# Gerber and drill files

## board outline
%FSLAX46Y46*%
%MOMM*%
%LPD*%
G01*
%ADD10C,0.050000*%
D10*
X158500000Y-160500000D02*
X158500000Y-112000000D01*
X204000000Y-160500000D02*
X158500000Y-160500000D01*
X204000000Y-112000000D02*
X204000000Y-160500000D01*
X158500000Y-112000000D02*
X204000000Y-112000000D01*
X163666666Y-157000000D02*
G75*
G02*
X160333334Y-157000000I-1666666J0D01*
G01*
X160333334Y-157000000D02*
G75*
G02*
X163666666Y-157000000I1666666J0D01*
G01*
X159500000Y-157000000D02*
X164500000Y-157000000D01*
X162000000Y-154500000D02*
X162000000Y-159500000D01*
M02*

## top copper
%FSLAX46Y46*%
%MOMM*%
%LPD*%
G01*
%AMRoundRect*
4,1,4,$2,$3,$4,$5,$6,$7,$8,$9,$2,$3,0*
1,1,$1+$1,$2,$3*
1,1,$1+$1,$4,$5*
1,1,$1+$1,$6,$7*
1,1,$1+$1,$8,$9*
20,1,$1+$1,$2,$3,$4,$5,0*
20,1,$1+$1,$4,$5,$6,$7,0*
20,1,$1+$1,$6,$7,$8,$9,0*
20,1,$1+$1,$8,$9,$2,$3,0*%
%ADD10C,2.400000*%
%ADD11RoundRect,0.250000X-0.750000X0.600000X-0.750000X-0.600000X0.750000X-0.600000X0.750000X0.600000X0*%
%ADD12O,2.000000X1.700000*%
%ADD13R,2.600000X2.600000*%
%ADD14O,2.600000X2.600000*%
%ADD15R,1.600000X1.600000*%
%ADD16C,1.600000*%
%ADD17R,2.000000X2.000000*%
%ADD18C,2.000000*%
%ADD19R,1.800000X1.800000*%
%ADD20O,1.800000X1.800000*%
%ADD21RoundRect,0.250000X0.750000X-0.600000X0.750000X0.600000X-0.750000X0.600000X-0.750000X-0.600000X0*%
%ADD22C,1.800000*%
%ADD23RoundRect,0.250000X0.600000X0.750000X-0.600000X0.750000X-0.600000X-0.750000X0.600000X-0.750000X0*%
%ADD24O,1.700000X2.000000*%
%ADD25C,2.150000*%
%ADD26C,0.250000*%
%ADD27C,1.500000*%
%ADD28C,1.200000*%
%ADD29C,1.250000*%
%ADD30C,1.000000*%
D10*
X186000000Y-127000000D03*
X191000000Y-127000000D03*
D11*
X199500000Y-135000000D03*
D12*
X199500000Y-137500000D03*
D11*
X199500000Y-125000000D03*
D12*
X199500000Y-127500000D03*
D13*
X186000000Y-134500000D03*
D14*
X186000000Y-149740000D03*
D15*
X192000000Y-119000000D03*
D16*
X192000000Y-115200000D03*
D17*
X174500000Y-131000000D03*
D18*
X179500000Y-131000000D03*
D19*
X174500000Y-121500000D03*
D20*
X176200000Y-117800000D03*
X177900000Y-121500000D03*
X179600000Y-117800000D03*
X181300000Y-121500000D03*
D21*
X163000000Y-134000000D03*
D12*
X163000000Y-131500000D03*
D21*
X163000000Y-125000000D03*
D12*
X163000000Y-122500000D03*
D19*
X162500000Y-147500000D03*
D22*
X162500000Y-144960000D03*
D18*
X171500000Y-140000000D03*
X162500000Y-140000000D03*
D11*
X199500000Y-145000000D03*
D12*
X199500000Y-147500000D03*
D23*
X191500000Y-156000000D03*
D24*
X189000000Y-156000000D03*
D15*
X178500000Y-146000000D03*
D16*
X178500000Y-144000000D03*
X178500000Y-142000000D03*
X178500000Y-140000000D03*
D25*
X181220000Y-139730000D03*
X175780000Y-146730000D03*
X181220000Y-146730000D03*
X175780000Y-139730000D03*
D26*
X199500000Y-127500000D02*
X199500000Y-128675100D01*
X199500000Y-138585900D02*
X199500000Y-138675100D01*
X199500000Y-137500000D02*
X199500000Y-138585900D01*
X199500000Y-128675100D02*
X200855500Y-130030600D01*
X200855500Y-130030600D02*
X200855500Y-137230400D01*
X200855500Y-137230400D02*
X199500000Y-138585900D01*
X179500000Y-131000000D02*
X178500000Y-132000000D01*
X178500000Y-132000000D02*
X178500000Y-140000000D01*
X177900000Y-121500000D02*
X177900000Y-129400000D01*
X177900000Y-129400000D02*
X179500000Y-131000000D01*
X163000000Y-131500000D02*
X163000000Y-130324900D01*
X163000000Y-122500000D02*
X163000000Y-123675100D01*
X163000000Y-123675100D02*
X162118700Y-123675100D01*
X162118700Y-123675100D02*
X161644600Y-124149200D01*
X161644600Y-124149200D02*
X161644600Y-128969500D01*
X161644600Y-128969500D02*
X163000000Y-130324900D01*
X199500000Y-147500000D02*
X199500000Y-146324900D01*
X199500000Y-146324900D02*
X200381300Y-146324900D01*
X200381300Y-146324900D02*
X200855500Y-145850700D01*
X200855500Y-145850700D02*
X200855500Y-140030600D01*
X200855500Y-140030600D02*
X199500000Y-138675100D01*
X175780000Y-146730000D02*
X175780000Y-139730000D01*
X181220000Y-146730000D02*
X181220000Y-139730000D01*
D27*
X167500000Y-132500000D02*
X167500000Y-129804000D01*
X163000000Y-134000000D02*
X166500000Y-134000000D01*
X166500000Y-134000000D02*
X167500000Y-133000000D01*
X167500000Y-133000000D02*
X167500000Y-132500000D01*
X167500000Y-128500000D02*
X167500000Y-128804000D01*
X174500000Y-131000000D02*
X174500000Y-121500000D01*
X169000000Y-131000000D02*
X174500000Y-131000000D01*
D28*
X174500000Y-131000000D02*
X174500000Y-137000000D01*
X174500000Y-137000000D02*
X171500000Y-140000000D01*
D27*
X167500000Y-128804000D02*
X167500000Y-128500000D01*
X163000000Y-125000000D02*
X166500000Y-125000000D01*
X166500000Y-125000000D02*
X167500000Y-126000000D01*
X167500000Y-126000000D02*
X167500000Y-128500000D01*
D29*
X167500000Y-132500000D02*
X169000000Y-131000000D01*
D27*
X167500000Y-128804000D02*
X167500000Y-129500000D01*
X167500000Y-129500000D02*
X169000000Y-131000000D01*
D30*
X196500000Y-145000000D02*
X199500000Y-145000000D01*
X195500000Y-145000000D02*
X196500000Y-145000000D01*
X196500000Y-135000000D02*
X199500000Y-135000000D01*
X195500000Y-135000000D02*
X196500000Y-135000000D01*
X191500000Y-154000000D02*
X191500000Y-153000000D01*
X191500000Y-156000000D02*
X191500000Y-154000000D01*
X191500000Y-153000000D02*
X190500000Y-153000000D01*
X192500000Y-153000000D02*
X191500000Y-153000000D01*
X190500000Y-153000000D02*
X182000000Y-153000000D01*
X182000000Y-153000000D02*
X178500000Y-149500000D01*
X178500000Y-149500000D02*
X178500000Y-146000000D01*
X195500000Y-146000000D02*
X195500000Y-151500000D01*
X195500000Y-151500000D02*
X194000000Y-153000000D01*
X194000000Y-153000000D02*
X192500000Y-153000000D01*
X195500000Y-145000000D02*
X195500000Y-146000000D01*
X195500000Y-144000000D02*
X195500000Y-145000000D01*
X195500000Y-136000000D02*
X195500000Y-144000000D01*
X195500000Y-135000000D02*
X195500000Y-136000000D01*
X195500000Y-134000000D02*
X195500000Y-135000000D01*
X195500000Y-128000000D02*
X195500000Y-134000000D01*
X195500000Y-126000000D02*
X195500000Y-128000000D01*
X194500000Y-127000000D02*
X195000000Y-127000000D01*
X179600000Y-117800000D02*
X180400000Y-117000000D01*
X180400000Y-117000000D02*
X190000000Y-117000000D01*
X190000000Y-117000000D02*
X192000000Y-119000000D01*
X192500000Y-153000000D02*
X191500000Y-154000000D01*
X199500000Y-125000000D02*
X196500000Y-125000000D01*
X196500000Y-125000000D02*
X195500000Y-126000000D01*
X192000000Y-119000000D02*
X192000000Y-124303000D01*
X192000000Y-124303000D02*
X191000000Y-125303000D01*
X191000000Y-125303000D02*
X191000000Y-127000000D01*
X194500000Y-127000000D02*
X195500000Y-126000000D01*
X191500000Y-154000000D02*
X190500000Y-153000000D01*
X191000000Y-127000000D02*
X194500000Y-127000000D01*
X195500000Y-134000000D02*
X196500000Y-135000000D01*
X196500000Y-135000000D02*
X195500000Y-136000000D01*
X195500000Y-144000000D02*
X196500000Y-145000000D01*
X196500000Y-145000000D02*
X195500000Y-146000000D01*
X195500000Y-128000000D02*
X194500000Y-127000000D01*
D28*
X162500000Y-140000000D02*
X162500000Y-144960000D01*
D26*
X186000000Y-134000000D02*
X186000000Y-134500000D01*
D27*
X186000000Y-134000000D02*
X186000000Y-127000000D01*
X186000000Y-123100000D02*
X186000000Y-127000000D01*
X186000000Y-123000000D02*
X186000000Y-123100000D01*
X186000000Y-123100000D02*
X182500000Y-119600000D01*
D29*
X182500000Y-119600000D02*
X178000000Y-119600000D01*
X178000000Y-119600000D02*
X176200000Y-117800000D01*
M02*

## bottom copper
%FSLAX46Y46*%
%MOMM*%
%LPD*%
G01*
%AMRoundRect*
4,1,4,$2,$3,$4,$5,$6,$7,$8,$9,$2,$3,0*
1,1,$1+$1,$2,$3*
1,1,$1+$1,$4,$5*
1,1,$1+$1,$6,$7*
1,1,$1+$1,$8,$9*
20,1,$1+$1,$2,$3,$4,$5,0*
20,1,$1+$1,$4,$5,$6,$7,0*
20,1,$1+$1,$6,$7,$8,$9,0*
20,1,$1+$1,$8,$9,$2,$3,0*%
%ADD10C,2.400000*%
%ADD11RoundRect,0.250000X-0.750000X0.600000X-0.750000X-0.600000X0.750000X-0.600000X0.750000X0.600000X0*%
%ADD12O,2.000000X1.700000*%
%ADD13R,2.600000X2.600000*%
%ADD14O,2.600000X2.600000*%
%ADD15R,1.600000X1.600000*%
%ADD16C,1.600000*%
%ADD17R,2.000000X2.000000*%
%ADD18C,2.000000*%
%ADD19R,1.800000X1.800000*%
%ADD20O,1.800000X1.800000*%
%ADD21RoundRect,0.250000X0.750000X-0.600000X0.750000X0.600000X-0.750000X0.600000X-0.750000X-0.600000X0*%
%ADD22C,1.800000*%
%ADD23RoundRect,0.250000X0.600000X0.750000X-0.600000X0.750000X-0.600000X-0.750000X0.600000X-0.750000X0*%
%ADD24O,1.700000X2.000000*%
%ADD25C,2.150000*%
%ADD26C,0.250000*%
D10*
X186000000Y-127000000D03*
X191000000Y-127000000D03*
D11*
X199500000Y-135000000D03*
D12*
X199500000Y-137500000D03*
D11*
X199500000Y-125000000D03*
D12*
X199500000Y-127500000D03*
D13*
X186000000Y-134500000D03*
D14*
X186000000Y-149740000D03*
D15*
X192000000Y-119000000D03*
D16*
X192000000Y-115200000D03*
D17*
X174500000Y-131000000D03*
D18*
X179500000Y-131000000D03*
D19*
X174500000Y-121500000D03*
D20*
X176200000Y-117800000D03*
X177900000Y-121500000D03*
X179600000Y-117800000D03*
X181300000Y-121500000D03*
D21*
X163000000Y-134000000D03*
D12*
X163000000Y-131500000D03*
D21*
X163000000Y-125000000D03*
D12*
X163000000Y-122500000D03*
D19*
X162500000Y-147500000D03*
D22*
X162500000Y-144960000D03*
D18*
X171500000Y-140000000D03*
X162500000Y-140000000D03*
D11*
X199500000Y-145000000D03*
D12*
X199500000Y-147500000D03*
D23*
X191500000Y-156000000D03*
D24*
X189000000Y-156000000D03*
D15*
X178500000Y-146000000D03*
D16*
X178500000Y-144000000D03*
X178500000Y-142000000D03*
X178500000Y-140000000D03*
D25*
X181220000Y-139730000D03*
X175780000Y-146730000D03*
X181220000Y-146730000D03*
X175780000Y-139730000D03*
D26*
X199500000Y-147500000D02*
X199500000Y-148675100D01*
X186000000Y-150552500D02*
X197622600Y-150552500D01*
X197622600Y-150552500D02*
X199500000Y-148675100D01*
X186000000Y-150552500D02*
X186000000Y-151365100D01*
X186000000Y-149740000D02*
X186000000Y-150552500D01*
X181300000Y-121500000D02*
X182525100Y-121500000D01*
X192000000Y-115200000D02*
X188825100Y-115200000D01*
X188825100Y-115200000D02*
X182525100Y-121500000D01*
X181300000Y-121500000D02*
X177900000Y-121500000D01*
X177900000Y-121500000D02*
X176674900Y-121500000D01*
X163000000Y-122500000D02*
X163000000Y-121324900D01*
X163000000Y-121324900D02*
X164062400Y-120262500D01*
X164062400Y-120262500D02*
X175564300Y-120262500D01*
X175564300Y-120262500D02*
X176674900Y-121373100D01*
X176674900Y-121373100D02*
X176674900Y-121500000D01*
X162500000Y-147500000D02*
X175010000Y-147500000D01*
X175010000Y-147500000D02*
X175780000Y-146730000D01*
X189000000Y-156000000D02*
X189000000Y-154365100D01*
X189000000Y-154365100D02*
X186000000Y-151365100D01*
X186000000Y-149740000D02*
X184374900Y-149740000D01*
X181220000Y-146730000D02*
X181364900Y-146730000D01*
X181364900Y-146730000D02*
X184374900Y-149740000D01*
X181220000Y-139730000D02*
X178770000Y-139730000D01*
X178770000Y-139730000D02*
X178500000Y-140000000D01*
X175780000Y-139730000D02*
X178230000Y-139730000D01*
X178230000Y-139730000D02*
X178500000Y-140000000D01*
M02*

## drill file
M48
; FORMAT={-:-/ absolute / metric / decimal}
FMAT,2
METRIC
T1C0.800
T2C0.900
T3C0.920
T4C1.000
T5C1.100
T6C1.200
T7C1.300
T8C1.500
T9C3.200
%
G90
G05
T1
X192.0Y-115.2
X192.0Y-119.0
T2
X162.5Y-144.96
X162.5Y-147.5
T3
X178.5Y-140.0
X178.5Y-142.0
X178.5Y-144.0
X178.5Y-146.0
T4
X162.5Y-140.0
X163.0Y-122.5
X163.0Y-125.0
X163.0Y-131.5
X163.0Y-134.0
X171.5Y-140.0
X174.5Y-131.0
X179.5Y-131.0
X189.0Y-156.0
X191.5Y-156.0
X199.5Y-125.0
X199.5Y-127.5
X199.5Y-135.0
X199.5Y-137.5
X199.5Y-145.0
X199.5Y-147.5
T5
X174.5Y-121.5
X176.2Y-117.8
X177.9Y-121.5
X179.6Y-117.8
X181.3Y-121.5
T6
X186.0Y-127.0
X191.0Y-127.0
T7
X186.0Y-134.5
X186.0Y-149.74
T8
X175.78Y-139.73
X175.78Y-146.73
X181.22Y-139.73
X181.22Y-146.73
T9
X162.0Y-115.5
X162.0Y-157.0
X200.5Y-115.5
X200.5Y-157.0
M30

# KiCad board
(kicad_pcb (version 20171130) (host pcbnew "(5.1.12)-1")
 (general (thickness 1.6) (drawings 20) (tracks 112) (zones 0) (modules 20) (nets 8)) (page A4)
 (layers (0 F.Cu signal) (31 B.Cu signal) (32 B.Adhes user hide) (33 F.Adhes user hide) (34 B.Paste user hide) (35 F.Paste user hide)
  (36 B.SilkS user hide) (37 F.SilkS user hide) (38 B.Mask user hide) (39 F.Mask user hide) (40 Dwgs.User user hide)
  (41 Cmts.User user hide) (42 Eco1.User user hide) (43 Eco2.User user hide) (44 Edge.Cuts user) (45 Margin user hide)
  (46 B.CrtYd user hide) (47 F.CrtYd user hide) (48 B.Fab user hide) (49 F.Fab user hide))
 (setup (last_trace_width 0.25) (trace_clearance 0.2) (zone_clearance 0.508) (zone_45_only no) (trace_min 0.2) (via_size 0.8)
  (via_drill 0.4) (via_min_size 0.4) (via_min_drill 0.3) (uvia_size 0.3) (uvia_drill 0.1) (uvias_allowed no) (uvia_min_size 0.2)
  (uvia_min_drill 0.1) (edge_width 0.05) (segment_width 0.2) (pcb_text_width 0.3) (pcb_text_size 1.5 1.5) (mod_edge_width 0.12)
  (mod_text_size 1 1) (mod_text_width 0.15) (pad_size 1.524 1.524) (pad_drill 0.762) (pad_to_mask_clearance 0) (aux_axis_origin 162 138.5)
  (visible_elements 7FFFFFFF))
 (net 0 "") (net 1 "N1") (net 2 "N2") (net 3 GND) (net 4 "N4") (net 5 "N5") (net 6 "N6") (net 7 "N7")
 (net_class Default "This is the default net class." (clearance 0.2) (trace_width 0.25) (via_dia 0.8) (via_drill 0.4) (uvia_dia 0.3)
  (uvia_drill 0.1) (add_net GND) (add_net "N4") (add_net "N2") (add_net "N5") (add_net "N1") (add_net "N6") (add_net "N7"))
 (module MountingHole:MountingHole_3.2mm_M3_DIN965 (layer F.Cu) (at 162 115.5)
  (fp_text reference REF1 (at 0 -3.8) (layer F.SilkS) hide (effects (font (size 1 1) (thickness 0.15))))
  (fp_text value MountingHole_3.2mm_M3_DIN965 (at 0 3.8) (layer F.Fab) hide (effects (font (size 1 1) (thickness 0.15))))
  (pad "" np_thru_hole circle (at 0 0) (size 3.2 3.2) (drill 3.2) (layers *.Cu *.Mask)))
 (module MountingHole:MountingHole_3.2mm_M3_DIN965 (layer F.Cu) (at 162 157)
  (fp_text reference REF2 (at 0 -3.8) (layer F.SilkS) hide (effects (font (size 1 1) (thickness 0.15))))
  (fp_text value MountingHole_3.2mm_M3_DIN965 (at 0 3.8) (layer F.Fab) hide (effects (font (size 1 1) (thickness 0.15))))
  (pad "" np_thru_hole circle (at 0 0) (size 3.2 3.2) (drill 3.2) (layers *.Cu *.Mask)))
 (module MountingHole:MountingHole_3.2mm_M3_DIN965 (layer F.Cu) (at 200.5 157)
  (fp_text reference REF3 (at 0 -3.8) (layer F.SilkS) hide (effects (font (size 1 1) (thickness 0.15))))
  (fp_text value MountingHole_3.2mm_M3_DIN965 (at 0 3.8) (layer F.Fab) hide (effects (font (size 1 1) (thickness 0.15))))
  (pad "" np_thru_hole circle (at 0 0) (size 3.2 3.2) (drill 3.2) (layers *.Cu *.Mask)))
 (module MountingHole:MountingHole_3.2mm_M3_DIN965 (layer F.Cu) (at 200.5 115.5)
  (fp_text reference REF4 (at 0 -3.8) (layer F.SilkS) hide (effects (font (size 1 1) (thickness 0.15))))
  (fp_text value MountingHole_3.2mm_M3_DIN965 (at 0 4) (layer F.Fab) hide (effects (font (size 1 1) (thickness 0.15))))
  (pad "" np_thru_hole circle (at 0 0) (size 3.2 3.2) (drill 3.2) (layers *.Cu *.Mask)))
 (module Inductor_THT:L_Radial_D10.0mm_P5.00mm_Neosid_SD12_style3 (layer F.Cu) (at 186 127)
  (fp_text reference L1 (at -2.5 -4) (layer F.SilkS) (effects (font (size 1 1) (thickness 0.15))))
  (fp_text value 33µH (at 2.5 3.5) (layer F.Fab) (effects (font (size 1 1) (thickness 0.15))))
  (pad 1 thru_hole circle (at 0 0) (size 2.4 2.4) (drill 1.2) (layers *.Cu *.Mask) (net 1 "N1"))
  (pad 2 thru_hole circle (at 5 0) (size 2.4 2.4) (drill 1.2) (layers *.Cu *.Mask) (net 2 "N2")))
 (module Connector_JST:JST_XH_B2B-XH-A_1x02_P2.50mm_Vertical (layer F.Cu) (at 199.5 135 270)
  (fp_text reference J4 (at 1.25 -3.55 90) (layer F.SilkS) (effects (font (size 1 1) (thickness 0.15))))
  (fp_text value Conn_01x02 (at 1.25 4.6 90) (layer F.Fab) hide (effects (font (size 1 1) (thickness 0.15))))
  (pad 1 thru_hole roundrect (at 0 0 270) (size 1.7 2) (drill 1) (layers *.Cu *.Mask) (roundrect_rratio 0.147059) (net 2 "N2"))
  (pad 2 thru_hole oval (at 2.5 0 270) (size 1.7 2) (drill 1) (layers *.Cu *.Mask) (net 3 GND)))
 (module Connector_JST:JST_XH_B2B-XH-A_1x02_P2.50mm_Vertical (layer F.Cu) (at 199.5 125 270)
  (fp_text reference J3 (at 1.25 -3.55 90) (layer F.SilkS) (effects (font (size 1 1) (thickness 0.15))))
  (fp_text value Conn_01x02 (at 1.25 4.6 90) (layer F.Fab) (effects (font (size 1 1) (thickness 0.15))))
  (pad 1 thru_hole roundrect (at 0 0 270) (size 1.7 2) (drill 1) (layers *.Cu *.Mask) (roundrect_rratio 0.147059) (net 2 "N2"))
  (pad 2 thru_hole oval (at 2.5 0 270) (size 1.7 2) (drill 1) (layers *.Cu *.Mask) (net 3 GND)))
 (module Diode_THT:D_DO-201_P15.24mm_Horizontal (layer F.Cu) (at 186 134.5 270)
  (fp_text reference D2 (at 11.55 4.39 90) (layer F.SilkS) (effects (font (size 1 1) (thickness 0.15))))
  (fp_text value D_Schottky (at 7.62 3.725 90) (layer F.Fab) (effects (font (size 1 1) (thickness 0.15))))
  (pad 1 thru_hole rect (at 0 0 270) (size 2.6 2.6) (drill 1.3) (layers *.Cu *.Mask) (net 1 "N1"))
  (pad 2 thru_hole oval (at 15.24 0 270) (size 2.6 2.6) (drill 1.3) (layers *.Cu *.Mask) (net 3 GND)))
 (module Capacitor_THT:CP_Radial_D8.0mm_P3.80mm (layer F.Cu) (at 192 119 90)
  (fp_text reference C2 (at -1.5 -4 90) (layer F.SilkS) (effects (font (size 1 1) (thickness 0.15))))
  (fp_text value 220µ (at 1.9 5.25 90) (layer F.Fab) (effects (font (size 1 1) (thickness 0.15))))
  (pad 1 thru_hole rect (at 0 0 90) (size 1.6 1.6) (drill 0.8) (layers *.Cu *.Mask) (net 2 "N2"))
  (pad 2 thru_hole circle (at 3.8 0 90) (size 1.6 1.6) (drill 0.8) (layers *.Cu *.Mask) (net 3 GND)))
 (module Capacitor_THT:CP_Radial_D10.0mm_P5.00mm (layer F.Cu) (at 174.5 131)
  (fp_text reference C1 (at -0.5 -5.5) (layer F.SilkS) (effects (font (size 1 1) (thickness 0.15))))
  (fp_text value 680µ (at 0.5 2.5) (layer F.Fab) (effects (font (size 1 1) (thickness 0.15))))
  (pad 1 thru_hole rect (at 0 0) (size 2 2) (drill 1) (layers *.Cu *.Mask) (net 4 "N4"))
  (pad 2 thru_hole circle (at 5 0) (size 2 2) (drill 1) (layers *.Cu *.Mask) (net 3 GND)))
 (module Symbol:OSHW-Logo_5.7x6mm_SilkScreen (layer F.Cu) (at 169 116.5)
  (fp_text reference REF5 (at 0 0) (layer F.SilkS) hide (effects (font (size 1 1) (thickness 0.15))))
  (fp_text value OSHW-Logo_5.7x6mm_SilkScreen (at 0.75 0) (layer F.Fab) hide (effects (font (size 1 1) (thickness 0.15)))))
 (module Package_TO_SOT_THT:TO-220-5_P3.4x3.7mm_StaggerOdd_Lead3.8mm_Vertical (layer F.Cu) (at 174.5 121.5)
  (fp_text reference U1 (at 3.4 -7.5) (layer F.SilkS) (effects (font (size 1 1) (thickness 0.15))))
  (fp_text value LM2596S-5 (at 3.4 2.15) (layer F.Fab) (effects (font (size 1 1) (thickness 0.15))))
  (pad 1 thru_hole rect (at 0 0) (size 1.8 1.8) (drill 1.1) (layers *.Cu *.Mask) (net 4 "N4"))
  (pad 2 thru_hole oval (at 1.7 -3.7) (size 1.8 1.8) (drill 1.1) (layers *.Cu *.Mask) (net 1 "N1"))
  (pad 3 thru_hole oval (at 3.4 0) (size 1.8 1.8) (drill 1.1) (layers *.Cu *.Mask) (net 3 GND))
  (pad 4 thru_hole oval (at 5.1 -3.7) (size 1.8 1.8) (drill 1.1) (layers *.Cu *.Mask) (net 2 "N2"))
  (pad 5 thru_hole oval (at 6.8 0) (size 1.8 1.8) (drill 1.1) (layers *.Cu *.Mask) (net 3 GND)))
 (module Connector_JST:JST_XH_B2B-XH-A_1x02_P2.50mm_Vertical (layer F.Cu) (at 163 134 90)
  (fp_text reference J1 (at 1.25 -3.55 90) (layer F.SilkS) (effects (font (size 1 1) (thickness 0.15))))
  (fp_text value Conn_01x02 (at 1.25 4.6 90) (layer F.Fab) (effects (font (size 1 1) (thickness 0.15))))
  (pad 1 thru_hole roundrect (at 0 0 90) (size 1.7 2) (drill 1) (layers *.Cu *.Mask) (roundrect_rratio 0.147059) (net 4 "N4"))
  (pad 2 thru_hole oval (at 2.5 0 90) (size 1.7 2) (drill 1) (layers *.Cu *.Mask) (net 3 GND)))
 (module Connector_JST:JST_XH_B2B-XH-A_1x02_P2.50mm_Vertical (layer F.Cu) (at 163 125 90)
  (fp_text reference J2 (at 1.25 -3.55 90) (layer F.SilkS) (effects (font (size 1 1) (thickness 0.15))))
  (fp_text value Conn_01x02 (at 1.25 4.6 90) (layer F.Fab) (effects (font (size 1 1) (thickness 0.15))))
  (pad 1 thru_hole roundrect (at 0 0 90) (size 1.7 2) (drill 1) (layers *.Cu *.Mask) (roundrect_rratio 0.147059) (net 4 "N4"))
  (pad 2 thru_hole oval (at 2.5 0 90) (size 1.7 2) (drill 1) (layers *.Cu *.Mask) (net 3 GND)))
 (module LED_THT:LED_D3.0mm (layer F.Cu) (at 162.5 147.5 90)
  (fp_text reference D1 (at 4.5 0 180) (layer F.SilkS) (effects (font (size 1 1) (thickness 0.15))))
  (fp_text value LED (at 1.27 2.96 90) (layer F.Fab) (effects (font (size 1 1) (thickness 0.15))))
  (pad 1 thru_hole rect (at 0 0 90) (size 1.8 1.8) (drill 0.9) (layers *.Cu *.Mask) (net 3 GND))
  (pad 2 thru_hole circle (at 2.54 0 90) (size 1.8 1.8) (drill 0.9) (layers *.Cu *.Mask) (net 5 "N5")))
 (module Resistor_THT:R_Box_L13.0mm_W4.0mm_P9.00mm (layer F.Cu) (at 171.5 140 180)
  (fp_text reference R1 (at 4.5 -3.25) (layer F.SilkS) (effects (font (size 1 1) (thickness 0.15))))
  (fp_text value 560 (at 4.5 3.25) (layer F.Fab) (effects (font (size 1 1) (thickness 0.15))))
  (pad 1 thru_hole circle (at 0 0 180) (size 2 2) (drill 1) (layers *.Cu *.Mask) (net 4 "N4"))
  (pad 2 thru_hole circle (at 9 0 180) (size 2 2) (drill 1) (layers *.Cu *.Mask) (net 5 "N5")))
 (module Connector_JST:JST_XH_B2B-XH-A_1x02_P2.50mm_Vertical (layer F.Cu) (at 199.5 145 270)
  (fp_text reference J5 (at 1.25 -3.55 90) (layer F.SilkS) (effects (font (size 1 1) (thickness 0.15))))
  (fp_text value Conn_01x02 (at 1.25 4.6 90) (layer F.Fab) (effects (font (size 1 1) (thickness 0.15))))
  (pad 1 thru_hole roundrect (at 0 0 270) (size 1.7 2) (drill 1) (layers *.Cu *.Mask) (roundrect_rratio 0.147059) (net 2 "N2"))
  (pad 2 thru_hole oval (at 2.5 0 270) (size 1.7 2) (drill 1) (layers *.Cu *.Mask) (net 3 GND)))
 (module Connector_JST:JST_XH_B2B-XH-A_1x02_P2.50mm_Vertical (layer F.Cu) (at 191.5 156 180)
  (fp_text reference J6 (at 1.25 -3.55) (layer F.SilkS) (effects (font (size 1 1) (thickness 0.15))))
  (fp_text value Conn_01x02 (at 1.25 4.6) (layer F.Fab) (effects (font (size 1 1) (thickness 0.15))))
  (pad 1 thru_hole roundrect (at 0 0 180) (size 1.7 2) (drill 1) (layers *.Cu *.Mask) (roundrect_rratio 0.147059) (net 2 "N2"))
  (pad 2 thru_hole oval (at 2.5 0 180) (size 1.7 2) (drill 1) (layers *.Cu *.Mask) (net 3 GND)))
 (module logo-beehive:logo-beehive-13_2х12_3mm (layer F.Cu) (at 170.5 151)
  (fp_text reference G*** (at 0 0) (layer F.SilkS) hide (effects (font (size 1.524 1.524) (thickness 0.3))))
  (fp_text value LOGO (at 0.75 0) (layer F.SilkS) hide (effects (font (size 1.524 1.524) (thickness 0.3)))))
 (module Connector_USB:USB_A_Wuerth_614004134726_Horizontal (layer F.Cu) (at 178.5 146 90)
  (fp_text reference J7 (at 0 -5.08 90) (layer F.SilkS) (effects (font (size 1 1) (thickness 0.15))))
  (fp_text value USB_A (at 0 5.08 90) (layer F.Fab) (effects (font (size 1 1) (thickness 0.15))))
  (pad 1 thru_hole rect (at 0 0 90) (size 1.6 1.6) (drill 0.92) (layers *.Cu *.Mask) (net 2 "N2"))
  (pad 2 thru_hole circle (at 2 0 90) (size 1.6 1.6) (drill 0.92) (layers *.Cu *.Mask) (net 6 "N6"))
  (pad 3 thru_hole circle (at 4 0 90) (size 1.6 1.6) (drill 0.92) (layers *.Cu *.Mask) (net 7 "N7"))
  (pad 4 thru_hole circle (at 6 0 90) (size 1.6 1.6) (drill 0.92) (layers *.Cu *.Mask) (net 3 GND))
  (pad 5 thru_hole circle (at 6.27 2.72 90) (size 2.15 2.15) (drill 1.5) (layers *.Cu *.Mask) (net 3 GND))
  (pad 5 thru_hole circle (at -0.73 -2.72 90) (size 2.15 2.15) (drill 1.5) (layers *.Cu *.Mask) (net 3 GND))
  (pad 5 thru_hole circle (at -0.73 2.72 90) (size 2.15 2.15) (drill 1.5) (layers *.Cu *.Mask) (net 3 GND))
  (pad 5 thru_hole circle (at 6.27 -2.72 90) (size 2.15 2.15) (drill 1.5) (layers *.Cu *.Mask) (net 3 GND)))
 (gr_line (start 158.5 160.5) (end 158.5 112) (layer Edge.Cuts) (width 0.05))
 (gr_line (start 204 160.5) (end 158.5 160.5) (layer Edge.Cuts) (width 0.05))
 (gr_line (start 204 112) (end 204 160.5) (layer Edge.Cuts) (width 0.05))
 (gr_line (start 158.5 112) (end 204 112) (layer Edge.Cuts) (width 0.05))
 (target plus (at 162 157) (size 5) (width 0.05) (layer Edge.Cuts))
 (segment (start 199.5 127.5) (end 199.5 128.6751) (width 0.25) (layer F.Cu) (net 3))
 (segment (start 199.5 138.5859) (end 199.5 138.6751) (width 0.25) (layer F.Cu) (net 3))
 (segment (start 199.5 137.5) (end 199.5 138.5859) (width 0.25) (layer F.Cu) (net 3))
 (segment (start 199.5 128.6751) (end 200.8555 130.0306) (width 0.25) (layer F.Cu) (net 3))
 (segment (start 200.8555 130.0306) (end 200.8555 137.2304) (width 0.25) (layer F.Cu) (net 3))
 (segment (start 200.8555 137.2304) (end 199.5 138.5859) (width 0.25) (layer F.Cu) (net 3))
 (segment (start 199.5 147.5) (end 199.5 148.6751) (width 0.25) (layer B.Cu) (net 3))
 (segment (start 186 150.5525) (end 197.6226 150.5525) (width 0.25) (layer B.Cu) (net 3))
 (segment (start 197.6226 150.5525) (end 199.5 148.6751) (width 0.25) (layer B.Cu) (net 3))
 (segment (start 186 150.5525) (end 186 151.3651) (width 0.25) (layer B.Cu) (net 3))
 (segment (start 186 149.74) (end 186 150.5525) (width 0.25) (layer B.Cu) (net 3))
 (segment (start 181.3 121.5) (end 182.5251 121.5) (width 0.25) (layer B.Cu) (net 3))
 (segment (start 192 115.2) (end 188.8251 115.2) (width 0.25) (layer B.Cu) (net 3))
 (segment (start 188.8251 115.2) (end 182.5251 121.5) (width 0.25) (layer B.Cu) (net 3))
 (segment (start 179.5 131) (end 178.5 132) (width 0.25) (layer F.Cu) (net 3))
 (segment (start 178.5 132) (end 178.5 140) (width 0.25) (layer F.Cu) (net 3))
 (segment (start 177.9 121.5) (end 177.9 129.4) (width 0.25) (layer F.Cu) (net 3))
 (segment (start 177.9 129.4) (end 179.5 131) (width 0.25) (layer F.Cu) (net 3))
 (segment (start 181.3 121.5) (end 177.9 121.5) (width 0.25) (layer B.Cu) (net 3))
 (segment (start 177.9 121.5) (end 176.6749 121.5) (width 0.25) (layer B.Cu) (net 3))
 (segment (start 163 122.5) (end 163 121.3249) (width 0.25) (layer B.Cu) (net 3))
 (segment (start 163 121.3249) (end 164.0624 120.2625) (width 0.25) (layer B.Cu) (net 3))
 (segment (start 164.0624 120.2625) (end 175.5643 120.2625) (width 0.25) (layer B.Cu) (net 3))
 (segment (start 175.5643 120.2625) (end 176.6749 121.3731) (width 0.25) (layer B.Cu) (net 3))
 (segment (start 176.6749 121.3731) (end 176.6749 121.5) (width 0.25) (layer B.Cu) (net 3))
 (segment (start 163 131.5) (end 163 130.3249) (width 0.25) (layer F.Cu) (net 3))
 (segment (start 163 122.5) (end 163 123.6751) (width 0.25) (layer F.Cu) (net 3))
 (segment (start 163 123.6751) (end 162.1187 123.6751) (width 0.25) (layer F.Cu) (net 3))
 (segment (start 162.1187 123.6751) (end 161.6446 124.1492) (width 0.25) (layer F.Cu) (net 3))
 (segment (start 161.6446 124.1492) (end 161.6446 128.9695) (width 0.25) (layer F.Cu) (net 3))
 (segment (start 161.6446 128.9695) (end 163 130.3249) (width 0.25) (layer F.Cu) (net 3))
 (segment (start 162.5 147.5) (end 175.01 147.5) (width 0.25) (layer B.Cu) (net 3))
 (segment (start 175.01 147.5) (end 175.78 146.73) (width 0.25) (layer B.Cu) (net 3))
 (segment (start 199.5 147.5) (end 199.5 146.3249) (width 0.25) (layer F.Cu) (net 3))
 (segment (start 199.5 146.3249) (end 200.3813 146.3249) (width 0.25) (layer F.Cu) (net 3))
 (segment (start 200.3813 146.3249) (end 200.8555 145.8507) (width 0.25) (layer F.Cu) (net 3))
 (segment (start 200.8555 145.8507) (end 200.8555 140.0306) (width 0.25) (layer F.Cu) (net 3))
 (segment (start 200.8555 140.0306) (end 199.5 138.6751) (width 0.25) (layer F.Cu) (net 3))
 (segment (start 189 156) (end 189 154.3651) (width 0.25) (layer B.Cu) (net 3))
 (segment (start 189 154.3651) (end 186 151.3651) (width 0.25) (layer B.Cu) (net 3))
 (segment (start 186 149.74) (end 184.3749 149.74) (width 0.25) (layer B.Cu) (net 3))
 (segment (start 181.22 146.73) (end 181.3649 146.73) (width 0.25) (layer B.Cu) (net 3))
 (segment (start 181.3649 146.73) (end 184.3749 149.74) (width 0.25) (layer B.Cu) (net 3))
 (segment (start 181.22 139.73) (end 178.77 139.73) (width 0.25) (layer B.Cu) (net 3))
 (segment (start 178.77 139.73) (end 178.5 140) (width 0.25) (layer B.Cu) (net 3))
 (segment (start 175.78 146.73) (end 175.78 139.73) (width 0.25) (layer F.Cu) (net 3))
 (segment (start 181.22 146.73) (end 181.22 139.73) (width 0.25) (layer F.Cu) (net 3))
 (segment (start 175.78 139.73) (end 178.23 139.73) (width 0.25) (layer B.Cu) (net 3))
 (segment (start 178.23 139.73) (end 178.5 140) (width 0.25) (layer B.Cu) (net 3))
 (segment (start 167.5 132.5) (end 167.5 129.804) (width 1.5) (layer F.Cu) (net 4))
 (segment (start 163 134) (end 166.5 134) (width 1.5) (layer F.Cu) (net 4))
 (segment (start 166.5 134) (end 167.5 133) (width 1.5) (layer F.Cu) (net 4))
 (segment (start 167.5 133) (end 167.5 132.5) (width 1.5) (layer F.Cu) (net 4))
 (segment (start 167.5 128.5) (end 167.5 128.804) (width 1.5) (layer F.Cu) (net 4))
 (segment (start 174.5 131) (end 174.5 121.5) (width 1.5) (layer F.Cu) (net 4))
 (segment (start 169 131) (end 174.5 131) (width 1.5) (layer F.Cu) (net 4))
 (segment (start 174.5 131) (end 174.5 137) (width 1.2) (layer F.Cu) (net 4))
 (segment (start 174.5 137) (end 171.5 140) (width 1.2) (layer F.Cu) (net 4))
 (segment (start 167.5 128.804) (end 167.5 128.5) (width 1.5) (layer F.Cu) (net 4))
 (segment (start 163 125) (end 166.5 125) (width 1.5) (layer F.Cu) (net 4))
 (segment (start 166.5 125) (end 167.5 126) (width 1.5) (layer F.Cu) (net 4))
 (segment (start 167.5 126) (end 167.5 128.5) (width 1.5) (layer F.Cu) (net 4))
 (segment (start 167.5 132.5) (end 169 131) (width 1.25) (layer F.Cu) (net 4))
 (segment (start 167.5 128.804) (end 167.5 129.5) (width 1.5) (layer F.Cu) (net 4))
 (segment (start 167.5 129.5) (end 169 131) (width 1.5) (layer F.Cu) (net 4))
 (segment (start 196.5 145) (end 199.5 145) (width 1) (layer F.Cu) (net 2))
 (segment (start 195.5 145) (end 196.5 145) (width 1) (layer F.Cu) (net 2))
 (segment (start 196.5 135) (end 199.5 135) (width 1) (layer F.Cu) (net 2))
 (segment (start 195.5 135) (end 196.5 135) (width 1) (layer F.Cu) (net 2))
 (segment (start 191.5 154) (end 191.5 153) (width 1) (layer F.Cu) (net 2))
 (segment (start 191.5 156) (end 191.5 154) (width 1) (layer F.Cu) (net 2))
 (segment (start 191.5 153) (end 190.5 153) (width 1) (layer F.Cu) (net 2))
 (segment (start 192.5 153) (end 191.5 153) (width 1) (layer F.Cu) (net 2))
 (segment (start 190.5 153) (end 182 153) (width 1) (layer F.Cu) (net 2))
 (segment (start 182 153) (end 178.5 149.5) (width 1) (layer F.Cu) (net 2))
 (segment (start 178.5 149.5) (end 178.5 146) (width 1) (layer F.Cu) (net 2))
 (segment (start 195.5 146) (end 195.5 151.5) (width 1) (layer F.Cu) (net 2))
 (segment (start 195.5 151.5) (end 194 153) (width 1) (layer F.Cu) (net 2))
 (segment (start 194 153) (end 192.5 153) (width 1) (layer F.Cu) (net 2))
 (segment (start 195.5 145) (end 195.5 146) (width 1) (layer F.Cu) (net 2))
 (segment (start 195.5 144) (end 195.5 145) (width 1) (layer F.Cu) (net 2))
 (segment (start 195.5 136) (end 195.5 144) (width 1) (layer F.Cu) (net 2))
 (segment (start 195.5 135) (end 195.5 136) (width 1) (layer F.Cu) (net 2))
 (segment (start 195.5 134) (end 195.5 135) (width 1) (layer F.Cu) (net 2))
 (segment (start 195.5 128) (end 195.5 134) (width 1) (layer F.Cu) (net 2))
 (segment (start 195.5 126) (end 195.5 128) (width 1) (layer F.Cu) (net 2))
 (segment (start 194.5 127) (end 195 127) (width 1) (layer F.Cu) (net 2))
 (segment (start 179.6 117.8) (end 180.4 117) (width 1) (layer F.Cu) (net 2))
 (segment (start 180.4 117) (end 190 117) (width 1) (layer F.Cu) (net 2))
 (segment (start 190 117) (end 192 119) (width 1) (layer F.Cu) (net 2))
 (segment (start 192.5 153) (end 191.5 154) (width 1) (layer F.Cu) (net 2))
 (segment (start 199.5 125) (end 196.5 125) (width 1) (layer F.Cu) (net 2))
 (segment (start 196.5 125) (end 195.5 126) (width 1) (layer F.Cu) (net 2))
 (segment (start 192 119) (end 192 124.303) (width 1) (layer F.Cu) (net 2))
 (segment (start 192 124.303) (end 191 125.303) (width 1) (layer F.Cu) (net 2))
 (segment (start 191 125.303) (end 191 127) (width 1) (layer F.Cu) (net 2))
 (segment (start 194.5 127) (end 195.5 126) (width 1) (layer F.Cu) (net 2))
 (segment (start 191.5 154) (end 190.5 153) (width 1) (layer F.Cu) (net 2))
 (segment (start 191 127) (end 194.5 127) (width 1) (layer F.Cu) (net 2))
 (segment (start 195.5 134) (end 196.5 135) (width 1) (layer F.Cu) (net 2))
 (segment (start 196.5 135) (end 195.5 136) (width 1) (layer F.Cu) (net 2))
 (segment (start 195.5 144) (end 196.5 145) (width 1) (layer F.Cu) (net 2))
 (segment (start 196.5 145) (end 195.5 146) (width 1) (layer F.Cu) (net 2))
 (segment (start 195.5 128) (end 194.5 127) (width 1) (layer F.Cu) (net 2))
 (segment (start 162.5 140) (end 162.5 144.96) (width 1.2) (layer F.Cu) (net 5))
 (segment (start 186 134) (end 186 134.5) (width 0.25) (layer F.Cu) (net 1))
 (segment (start 186 134) (end 186 127) (width 1.5) (layer F.Cu) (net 1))
 (segment (start 186 123.1) (end 186 127) (width 1.5) (layer F.Cu) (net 1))
 (segment (start 186 123) (end 186 123.1) (width 1.5) (layer F.Cu) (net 1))
 (segment (start 186 123.1) (end 182.5 119.6) (width 1.5) (layer F.Cu) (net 1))
 (segment (start 182.5 119.6) (end 178 119.6) (width 1.25) (layer F.Cu) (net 1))
 (segment (start 178 119.6) (end 176.2 117.8) (width 1.25) (layer F.Cu) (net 1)))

